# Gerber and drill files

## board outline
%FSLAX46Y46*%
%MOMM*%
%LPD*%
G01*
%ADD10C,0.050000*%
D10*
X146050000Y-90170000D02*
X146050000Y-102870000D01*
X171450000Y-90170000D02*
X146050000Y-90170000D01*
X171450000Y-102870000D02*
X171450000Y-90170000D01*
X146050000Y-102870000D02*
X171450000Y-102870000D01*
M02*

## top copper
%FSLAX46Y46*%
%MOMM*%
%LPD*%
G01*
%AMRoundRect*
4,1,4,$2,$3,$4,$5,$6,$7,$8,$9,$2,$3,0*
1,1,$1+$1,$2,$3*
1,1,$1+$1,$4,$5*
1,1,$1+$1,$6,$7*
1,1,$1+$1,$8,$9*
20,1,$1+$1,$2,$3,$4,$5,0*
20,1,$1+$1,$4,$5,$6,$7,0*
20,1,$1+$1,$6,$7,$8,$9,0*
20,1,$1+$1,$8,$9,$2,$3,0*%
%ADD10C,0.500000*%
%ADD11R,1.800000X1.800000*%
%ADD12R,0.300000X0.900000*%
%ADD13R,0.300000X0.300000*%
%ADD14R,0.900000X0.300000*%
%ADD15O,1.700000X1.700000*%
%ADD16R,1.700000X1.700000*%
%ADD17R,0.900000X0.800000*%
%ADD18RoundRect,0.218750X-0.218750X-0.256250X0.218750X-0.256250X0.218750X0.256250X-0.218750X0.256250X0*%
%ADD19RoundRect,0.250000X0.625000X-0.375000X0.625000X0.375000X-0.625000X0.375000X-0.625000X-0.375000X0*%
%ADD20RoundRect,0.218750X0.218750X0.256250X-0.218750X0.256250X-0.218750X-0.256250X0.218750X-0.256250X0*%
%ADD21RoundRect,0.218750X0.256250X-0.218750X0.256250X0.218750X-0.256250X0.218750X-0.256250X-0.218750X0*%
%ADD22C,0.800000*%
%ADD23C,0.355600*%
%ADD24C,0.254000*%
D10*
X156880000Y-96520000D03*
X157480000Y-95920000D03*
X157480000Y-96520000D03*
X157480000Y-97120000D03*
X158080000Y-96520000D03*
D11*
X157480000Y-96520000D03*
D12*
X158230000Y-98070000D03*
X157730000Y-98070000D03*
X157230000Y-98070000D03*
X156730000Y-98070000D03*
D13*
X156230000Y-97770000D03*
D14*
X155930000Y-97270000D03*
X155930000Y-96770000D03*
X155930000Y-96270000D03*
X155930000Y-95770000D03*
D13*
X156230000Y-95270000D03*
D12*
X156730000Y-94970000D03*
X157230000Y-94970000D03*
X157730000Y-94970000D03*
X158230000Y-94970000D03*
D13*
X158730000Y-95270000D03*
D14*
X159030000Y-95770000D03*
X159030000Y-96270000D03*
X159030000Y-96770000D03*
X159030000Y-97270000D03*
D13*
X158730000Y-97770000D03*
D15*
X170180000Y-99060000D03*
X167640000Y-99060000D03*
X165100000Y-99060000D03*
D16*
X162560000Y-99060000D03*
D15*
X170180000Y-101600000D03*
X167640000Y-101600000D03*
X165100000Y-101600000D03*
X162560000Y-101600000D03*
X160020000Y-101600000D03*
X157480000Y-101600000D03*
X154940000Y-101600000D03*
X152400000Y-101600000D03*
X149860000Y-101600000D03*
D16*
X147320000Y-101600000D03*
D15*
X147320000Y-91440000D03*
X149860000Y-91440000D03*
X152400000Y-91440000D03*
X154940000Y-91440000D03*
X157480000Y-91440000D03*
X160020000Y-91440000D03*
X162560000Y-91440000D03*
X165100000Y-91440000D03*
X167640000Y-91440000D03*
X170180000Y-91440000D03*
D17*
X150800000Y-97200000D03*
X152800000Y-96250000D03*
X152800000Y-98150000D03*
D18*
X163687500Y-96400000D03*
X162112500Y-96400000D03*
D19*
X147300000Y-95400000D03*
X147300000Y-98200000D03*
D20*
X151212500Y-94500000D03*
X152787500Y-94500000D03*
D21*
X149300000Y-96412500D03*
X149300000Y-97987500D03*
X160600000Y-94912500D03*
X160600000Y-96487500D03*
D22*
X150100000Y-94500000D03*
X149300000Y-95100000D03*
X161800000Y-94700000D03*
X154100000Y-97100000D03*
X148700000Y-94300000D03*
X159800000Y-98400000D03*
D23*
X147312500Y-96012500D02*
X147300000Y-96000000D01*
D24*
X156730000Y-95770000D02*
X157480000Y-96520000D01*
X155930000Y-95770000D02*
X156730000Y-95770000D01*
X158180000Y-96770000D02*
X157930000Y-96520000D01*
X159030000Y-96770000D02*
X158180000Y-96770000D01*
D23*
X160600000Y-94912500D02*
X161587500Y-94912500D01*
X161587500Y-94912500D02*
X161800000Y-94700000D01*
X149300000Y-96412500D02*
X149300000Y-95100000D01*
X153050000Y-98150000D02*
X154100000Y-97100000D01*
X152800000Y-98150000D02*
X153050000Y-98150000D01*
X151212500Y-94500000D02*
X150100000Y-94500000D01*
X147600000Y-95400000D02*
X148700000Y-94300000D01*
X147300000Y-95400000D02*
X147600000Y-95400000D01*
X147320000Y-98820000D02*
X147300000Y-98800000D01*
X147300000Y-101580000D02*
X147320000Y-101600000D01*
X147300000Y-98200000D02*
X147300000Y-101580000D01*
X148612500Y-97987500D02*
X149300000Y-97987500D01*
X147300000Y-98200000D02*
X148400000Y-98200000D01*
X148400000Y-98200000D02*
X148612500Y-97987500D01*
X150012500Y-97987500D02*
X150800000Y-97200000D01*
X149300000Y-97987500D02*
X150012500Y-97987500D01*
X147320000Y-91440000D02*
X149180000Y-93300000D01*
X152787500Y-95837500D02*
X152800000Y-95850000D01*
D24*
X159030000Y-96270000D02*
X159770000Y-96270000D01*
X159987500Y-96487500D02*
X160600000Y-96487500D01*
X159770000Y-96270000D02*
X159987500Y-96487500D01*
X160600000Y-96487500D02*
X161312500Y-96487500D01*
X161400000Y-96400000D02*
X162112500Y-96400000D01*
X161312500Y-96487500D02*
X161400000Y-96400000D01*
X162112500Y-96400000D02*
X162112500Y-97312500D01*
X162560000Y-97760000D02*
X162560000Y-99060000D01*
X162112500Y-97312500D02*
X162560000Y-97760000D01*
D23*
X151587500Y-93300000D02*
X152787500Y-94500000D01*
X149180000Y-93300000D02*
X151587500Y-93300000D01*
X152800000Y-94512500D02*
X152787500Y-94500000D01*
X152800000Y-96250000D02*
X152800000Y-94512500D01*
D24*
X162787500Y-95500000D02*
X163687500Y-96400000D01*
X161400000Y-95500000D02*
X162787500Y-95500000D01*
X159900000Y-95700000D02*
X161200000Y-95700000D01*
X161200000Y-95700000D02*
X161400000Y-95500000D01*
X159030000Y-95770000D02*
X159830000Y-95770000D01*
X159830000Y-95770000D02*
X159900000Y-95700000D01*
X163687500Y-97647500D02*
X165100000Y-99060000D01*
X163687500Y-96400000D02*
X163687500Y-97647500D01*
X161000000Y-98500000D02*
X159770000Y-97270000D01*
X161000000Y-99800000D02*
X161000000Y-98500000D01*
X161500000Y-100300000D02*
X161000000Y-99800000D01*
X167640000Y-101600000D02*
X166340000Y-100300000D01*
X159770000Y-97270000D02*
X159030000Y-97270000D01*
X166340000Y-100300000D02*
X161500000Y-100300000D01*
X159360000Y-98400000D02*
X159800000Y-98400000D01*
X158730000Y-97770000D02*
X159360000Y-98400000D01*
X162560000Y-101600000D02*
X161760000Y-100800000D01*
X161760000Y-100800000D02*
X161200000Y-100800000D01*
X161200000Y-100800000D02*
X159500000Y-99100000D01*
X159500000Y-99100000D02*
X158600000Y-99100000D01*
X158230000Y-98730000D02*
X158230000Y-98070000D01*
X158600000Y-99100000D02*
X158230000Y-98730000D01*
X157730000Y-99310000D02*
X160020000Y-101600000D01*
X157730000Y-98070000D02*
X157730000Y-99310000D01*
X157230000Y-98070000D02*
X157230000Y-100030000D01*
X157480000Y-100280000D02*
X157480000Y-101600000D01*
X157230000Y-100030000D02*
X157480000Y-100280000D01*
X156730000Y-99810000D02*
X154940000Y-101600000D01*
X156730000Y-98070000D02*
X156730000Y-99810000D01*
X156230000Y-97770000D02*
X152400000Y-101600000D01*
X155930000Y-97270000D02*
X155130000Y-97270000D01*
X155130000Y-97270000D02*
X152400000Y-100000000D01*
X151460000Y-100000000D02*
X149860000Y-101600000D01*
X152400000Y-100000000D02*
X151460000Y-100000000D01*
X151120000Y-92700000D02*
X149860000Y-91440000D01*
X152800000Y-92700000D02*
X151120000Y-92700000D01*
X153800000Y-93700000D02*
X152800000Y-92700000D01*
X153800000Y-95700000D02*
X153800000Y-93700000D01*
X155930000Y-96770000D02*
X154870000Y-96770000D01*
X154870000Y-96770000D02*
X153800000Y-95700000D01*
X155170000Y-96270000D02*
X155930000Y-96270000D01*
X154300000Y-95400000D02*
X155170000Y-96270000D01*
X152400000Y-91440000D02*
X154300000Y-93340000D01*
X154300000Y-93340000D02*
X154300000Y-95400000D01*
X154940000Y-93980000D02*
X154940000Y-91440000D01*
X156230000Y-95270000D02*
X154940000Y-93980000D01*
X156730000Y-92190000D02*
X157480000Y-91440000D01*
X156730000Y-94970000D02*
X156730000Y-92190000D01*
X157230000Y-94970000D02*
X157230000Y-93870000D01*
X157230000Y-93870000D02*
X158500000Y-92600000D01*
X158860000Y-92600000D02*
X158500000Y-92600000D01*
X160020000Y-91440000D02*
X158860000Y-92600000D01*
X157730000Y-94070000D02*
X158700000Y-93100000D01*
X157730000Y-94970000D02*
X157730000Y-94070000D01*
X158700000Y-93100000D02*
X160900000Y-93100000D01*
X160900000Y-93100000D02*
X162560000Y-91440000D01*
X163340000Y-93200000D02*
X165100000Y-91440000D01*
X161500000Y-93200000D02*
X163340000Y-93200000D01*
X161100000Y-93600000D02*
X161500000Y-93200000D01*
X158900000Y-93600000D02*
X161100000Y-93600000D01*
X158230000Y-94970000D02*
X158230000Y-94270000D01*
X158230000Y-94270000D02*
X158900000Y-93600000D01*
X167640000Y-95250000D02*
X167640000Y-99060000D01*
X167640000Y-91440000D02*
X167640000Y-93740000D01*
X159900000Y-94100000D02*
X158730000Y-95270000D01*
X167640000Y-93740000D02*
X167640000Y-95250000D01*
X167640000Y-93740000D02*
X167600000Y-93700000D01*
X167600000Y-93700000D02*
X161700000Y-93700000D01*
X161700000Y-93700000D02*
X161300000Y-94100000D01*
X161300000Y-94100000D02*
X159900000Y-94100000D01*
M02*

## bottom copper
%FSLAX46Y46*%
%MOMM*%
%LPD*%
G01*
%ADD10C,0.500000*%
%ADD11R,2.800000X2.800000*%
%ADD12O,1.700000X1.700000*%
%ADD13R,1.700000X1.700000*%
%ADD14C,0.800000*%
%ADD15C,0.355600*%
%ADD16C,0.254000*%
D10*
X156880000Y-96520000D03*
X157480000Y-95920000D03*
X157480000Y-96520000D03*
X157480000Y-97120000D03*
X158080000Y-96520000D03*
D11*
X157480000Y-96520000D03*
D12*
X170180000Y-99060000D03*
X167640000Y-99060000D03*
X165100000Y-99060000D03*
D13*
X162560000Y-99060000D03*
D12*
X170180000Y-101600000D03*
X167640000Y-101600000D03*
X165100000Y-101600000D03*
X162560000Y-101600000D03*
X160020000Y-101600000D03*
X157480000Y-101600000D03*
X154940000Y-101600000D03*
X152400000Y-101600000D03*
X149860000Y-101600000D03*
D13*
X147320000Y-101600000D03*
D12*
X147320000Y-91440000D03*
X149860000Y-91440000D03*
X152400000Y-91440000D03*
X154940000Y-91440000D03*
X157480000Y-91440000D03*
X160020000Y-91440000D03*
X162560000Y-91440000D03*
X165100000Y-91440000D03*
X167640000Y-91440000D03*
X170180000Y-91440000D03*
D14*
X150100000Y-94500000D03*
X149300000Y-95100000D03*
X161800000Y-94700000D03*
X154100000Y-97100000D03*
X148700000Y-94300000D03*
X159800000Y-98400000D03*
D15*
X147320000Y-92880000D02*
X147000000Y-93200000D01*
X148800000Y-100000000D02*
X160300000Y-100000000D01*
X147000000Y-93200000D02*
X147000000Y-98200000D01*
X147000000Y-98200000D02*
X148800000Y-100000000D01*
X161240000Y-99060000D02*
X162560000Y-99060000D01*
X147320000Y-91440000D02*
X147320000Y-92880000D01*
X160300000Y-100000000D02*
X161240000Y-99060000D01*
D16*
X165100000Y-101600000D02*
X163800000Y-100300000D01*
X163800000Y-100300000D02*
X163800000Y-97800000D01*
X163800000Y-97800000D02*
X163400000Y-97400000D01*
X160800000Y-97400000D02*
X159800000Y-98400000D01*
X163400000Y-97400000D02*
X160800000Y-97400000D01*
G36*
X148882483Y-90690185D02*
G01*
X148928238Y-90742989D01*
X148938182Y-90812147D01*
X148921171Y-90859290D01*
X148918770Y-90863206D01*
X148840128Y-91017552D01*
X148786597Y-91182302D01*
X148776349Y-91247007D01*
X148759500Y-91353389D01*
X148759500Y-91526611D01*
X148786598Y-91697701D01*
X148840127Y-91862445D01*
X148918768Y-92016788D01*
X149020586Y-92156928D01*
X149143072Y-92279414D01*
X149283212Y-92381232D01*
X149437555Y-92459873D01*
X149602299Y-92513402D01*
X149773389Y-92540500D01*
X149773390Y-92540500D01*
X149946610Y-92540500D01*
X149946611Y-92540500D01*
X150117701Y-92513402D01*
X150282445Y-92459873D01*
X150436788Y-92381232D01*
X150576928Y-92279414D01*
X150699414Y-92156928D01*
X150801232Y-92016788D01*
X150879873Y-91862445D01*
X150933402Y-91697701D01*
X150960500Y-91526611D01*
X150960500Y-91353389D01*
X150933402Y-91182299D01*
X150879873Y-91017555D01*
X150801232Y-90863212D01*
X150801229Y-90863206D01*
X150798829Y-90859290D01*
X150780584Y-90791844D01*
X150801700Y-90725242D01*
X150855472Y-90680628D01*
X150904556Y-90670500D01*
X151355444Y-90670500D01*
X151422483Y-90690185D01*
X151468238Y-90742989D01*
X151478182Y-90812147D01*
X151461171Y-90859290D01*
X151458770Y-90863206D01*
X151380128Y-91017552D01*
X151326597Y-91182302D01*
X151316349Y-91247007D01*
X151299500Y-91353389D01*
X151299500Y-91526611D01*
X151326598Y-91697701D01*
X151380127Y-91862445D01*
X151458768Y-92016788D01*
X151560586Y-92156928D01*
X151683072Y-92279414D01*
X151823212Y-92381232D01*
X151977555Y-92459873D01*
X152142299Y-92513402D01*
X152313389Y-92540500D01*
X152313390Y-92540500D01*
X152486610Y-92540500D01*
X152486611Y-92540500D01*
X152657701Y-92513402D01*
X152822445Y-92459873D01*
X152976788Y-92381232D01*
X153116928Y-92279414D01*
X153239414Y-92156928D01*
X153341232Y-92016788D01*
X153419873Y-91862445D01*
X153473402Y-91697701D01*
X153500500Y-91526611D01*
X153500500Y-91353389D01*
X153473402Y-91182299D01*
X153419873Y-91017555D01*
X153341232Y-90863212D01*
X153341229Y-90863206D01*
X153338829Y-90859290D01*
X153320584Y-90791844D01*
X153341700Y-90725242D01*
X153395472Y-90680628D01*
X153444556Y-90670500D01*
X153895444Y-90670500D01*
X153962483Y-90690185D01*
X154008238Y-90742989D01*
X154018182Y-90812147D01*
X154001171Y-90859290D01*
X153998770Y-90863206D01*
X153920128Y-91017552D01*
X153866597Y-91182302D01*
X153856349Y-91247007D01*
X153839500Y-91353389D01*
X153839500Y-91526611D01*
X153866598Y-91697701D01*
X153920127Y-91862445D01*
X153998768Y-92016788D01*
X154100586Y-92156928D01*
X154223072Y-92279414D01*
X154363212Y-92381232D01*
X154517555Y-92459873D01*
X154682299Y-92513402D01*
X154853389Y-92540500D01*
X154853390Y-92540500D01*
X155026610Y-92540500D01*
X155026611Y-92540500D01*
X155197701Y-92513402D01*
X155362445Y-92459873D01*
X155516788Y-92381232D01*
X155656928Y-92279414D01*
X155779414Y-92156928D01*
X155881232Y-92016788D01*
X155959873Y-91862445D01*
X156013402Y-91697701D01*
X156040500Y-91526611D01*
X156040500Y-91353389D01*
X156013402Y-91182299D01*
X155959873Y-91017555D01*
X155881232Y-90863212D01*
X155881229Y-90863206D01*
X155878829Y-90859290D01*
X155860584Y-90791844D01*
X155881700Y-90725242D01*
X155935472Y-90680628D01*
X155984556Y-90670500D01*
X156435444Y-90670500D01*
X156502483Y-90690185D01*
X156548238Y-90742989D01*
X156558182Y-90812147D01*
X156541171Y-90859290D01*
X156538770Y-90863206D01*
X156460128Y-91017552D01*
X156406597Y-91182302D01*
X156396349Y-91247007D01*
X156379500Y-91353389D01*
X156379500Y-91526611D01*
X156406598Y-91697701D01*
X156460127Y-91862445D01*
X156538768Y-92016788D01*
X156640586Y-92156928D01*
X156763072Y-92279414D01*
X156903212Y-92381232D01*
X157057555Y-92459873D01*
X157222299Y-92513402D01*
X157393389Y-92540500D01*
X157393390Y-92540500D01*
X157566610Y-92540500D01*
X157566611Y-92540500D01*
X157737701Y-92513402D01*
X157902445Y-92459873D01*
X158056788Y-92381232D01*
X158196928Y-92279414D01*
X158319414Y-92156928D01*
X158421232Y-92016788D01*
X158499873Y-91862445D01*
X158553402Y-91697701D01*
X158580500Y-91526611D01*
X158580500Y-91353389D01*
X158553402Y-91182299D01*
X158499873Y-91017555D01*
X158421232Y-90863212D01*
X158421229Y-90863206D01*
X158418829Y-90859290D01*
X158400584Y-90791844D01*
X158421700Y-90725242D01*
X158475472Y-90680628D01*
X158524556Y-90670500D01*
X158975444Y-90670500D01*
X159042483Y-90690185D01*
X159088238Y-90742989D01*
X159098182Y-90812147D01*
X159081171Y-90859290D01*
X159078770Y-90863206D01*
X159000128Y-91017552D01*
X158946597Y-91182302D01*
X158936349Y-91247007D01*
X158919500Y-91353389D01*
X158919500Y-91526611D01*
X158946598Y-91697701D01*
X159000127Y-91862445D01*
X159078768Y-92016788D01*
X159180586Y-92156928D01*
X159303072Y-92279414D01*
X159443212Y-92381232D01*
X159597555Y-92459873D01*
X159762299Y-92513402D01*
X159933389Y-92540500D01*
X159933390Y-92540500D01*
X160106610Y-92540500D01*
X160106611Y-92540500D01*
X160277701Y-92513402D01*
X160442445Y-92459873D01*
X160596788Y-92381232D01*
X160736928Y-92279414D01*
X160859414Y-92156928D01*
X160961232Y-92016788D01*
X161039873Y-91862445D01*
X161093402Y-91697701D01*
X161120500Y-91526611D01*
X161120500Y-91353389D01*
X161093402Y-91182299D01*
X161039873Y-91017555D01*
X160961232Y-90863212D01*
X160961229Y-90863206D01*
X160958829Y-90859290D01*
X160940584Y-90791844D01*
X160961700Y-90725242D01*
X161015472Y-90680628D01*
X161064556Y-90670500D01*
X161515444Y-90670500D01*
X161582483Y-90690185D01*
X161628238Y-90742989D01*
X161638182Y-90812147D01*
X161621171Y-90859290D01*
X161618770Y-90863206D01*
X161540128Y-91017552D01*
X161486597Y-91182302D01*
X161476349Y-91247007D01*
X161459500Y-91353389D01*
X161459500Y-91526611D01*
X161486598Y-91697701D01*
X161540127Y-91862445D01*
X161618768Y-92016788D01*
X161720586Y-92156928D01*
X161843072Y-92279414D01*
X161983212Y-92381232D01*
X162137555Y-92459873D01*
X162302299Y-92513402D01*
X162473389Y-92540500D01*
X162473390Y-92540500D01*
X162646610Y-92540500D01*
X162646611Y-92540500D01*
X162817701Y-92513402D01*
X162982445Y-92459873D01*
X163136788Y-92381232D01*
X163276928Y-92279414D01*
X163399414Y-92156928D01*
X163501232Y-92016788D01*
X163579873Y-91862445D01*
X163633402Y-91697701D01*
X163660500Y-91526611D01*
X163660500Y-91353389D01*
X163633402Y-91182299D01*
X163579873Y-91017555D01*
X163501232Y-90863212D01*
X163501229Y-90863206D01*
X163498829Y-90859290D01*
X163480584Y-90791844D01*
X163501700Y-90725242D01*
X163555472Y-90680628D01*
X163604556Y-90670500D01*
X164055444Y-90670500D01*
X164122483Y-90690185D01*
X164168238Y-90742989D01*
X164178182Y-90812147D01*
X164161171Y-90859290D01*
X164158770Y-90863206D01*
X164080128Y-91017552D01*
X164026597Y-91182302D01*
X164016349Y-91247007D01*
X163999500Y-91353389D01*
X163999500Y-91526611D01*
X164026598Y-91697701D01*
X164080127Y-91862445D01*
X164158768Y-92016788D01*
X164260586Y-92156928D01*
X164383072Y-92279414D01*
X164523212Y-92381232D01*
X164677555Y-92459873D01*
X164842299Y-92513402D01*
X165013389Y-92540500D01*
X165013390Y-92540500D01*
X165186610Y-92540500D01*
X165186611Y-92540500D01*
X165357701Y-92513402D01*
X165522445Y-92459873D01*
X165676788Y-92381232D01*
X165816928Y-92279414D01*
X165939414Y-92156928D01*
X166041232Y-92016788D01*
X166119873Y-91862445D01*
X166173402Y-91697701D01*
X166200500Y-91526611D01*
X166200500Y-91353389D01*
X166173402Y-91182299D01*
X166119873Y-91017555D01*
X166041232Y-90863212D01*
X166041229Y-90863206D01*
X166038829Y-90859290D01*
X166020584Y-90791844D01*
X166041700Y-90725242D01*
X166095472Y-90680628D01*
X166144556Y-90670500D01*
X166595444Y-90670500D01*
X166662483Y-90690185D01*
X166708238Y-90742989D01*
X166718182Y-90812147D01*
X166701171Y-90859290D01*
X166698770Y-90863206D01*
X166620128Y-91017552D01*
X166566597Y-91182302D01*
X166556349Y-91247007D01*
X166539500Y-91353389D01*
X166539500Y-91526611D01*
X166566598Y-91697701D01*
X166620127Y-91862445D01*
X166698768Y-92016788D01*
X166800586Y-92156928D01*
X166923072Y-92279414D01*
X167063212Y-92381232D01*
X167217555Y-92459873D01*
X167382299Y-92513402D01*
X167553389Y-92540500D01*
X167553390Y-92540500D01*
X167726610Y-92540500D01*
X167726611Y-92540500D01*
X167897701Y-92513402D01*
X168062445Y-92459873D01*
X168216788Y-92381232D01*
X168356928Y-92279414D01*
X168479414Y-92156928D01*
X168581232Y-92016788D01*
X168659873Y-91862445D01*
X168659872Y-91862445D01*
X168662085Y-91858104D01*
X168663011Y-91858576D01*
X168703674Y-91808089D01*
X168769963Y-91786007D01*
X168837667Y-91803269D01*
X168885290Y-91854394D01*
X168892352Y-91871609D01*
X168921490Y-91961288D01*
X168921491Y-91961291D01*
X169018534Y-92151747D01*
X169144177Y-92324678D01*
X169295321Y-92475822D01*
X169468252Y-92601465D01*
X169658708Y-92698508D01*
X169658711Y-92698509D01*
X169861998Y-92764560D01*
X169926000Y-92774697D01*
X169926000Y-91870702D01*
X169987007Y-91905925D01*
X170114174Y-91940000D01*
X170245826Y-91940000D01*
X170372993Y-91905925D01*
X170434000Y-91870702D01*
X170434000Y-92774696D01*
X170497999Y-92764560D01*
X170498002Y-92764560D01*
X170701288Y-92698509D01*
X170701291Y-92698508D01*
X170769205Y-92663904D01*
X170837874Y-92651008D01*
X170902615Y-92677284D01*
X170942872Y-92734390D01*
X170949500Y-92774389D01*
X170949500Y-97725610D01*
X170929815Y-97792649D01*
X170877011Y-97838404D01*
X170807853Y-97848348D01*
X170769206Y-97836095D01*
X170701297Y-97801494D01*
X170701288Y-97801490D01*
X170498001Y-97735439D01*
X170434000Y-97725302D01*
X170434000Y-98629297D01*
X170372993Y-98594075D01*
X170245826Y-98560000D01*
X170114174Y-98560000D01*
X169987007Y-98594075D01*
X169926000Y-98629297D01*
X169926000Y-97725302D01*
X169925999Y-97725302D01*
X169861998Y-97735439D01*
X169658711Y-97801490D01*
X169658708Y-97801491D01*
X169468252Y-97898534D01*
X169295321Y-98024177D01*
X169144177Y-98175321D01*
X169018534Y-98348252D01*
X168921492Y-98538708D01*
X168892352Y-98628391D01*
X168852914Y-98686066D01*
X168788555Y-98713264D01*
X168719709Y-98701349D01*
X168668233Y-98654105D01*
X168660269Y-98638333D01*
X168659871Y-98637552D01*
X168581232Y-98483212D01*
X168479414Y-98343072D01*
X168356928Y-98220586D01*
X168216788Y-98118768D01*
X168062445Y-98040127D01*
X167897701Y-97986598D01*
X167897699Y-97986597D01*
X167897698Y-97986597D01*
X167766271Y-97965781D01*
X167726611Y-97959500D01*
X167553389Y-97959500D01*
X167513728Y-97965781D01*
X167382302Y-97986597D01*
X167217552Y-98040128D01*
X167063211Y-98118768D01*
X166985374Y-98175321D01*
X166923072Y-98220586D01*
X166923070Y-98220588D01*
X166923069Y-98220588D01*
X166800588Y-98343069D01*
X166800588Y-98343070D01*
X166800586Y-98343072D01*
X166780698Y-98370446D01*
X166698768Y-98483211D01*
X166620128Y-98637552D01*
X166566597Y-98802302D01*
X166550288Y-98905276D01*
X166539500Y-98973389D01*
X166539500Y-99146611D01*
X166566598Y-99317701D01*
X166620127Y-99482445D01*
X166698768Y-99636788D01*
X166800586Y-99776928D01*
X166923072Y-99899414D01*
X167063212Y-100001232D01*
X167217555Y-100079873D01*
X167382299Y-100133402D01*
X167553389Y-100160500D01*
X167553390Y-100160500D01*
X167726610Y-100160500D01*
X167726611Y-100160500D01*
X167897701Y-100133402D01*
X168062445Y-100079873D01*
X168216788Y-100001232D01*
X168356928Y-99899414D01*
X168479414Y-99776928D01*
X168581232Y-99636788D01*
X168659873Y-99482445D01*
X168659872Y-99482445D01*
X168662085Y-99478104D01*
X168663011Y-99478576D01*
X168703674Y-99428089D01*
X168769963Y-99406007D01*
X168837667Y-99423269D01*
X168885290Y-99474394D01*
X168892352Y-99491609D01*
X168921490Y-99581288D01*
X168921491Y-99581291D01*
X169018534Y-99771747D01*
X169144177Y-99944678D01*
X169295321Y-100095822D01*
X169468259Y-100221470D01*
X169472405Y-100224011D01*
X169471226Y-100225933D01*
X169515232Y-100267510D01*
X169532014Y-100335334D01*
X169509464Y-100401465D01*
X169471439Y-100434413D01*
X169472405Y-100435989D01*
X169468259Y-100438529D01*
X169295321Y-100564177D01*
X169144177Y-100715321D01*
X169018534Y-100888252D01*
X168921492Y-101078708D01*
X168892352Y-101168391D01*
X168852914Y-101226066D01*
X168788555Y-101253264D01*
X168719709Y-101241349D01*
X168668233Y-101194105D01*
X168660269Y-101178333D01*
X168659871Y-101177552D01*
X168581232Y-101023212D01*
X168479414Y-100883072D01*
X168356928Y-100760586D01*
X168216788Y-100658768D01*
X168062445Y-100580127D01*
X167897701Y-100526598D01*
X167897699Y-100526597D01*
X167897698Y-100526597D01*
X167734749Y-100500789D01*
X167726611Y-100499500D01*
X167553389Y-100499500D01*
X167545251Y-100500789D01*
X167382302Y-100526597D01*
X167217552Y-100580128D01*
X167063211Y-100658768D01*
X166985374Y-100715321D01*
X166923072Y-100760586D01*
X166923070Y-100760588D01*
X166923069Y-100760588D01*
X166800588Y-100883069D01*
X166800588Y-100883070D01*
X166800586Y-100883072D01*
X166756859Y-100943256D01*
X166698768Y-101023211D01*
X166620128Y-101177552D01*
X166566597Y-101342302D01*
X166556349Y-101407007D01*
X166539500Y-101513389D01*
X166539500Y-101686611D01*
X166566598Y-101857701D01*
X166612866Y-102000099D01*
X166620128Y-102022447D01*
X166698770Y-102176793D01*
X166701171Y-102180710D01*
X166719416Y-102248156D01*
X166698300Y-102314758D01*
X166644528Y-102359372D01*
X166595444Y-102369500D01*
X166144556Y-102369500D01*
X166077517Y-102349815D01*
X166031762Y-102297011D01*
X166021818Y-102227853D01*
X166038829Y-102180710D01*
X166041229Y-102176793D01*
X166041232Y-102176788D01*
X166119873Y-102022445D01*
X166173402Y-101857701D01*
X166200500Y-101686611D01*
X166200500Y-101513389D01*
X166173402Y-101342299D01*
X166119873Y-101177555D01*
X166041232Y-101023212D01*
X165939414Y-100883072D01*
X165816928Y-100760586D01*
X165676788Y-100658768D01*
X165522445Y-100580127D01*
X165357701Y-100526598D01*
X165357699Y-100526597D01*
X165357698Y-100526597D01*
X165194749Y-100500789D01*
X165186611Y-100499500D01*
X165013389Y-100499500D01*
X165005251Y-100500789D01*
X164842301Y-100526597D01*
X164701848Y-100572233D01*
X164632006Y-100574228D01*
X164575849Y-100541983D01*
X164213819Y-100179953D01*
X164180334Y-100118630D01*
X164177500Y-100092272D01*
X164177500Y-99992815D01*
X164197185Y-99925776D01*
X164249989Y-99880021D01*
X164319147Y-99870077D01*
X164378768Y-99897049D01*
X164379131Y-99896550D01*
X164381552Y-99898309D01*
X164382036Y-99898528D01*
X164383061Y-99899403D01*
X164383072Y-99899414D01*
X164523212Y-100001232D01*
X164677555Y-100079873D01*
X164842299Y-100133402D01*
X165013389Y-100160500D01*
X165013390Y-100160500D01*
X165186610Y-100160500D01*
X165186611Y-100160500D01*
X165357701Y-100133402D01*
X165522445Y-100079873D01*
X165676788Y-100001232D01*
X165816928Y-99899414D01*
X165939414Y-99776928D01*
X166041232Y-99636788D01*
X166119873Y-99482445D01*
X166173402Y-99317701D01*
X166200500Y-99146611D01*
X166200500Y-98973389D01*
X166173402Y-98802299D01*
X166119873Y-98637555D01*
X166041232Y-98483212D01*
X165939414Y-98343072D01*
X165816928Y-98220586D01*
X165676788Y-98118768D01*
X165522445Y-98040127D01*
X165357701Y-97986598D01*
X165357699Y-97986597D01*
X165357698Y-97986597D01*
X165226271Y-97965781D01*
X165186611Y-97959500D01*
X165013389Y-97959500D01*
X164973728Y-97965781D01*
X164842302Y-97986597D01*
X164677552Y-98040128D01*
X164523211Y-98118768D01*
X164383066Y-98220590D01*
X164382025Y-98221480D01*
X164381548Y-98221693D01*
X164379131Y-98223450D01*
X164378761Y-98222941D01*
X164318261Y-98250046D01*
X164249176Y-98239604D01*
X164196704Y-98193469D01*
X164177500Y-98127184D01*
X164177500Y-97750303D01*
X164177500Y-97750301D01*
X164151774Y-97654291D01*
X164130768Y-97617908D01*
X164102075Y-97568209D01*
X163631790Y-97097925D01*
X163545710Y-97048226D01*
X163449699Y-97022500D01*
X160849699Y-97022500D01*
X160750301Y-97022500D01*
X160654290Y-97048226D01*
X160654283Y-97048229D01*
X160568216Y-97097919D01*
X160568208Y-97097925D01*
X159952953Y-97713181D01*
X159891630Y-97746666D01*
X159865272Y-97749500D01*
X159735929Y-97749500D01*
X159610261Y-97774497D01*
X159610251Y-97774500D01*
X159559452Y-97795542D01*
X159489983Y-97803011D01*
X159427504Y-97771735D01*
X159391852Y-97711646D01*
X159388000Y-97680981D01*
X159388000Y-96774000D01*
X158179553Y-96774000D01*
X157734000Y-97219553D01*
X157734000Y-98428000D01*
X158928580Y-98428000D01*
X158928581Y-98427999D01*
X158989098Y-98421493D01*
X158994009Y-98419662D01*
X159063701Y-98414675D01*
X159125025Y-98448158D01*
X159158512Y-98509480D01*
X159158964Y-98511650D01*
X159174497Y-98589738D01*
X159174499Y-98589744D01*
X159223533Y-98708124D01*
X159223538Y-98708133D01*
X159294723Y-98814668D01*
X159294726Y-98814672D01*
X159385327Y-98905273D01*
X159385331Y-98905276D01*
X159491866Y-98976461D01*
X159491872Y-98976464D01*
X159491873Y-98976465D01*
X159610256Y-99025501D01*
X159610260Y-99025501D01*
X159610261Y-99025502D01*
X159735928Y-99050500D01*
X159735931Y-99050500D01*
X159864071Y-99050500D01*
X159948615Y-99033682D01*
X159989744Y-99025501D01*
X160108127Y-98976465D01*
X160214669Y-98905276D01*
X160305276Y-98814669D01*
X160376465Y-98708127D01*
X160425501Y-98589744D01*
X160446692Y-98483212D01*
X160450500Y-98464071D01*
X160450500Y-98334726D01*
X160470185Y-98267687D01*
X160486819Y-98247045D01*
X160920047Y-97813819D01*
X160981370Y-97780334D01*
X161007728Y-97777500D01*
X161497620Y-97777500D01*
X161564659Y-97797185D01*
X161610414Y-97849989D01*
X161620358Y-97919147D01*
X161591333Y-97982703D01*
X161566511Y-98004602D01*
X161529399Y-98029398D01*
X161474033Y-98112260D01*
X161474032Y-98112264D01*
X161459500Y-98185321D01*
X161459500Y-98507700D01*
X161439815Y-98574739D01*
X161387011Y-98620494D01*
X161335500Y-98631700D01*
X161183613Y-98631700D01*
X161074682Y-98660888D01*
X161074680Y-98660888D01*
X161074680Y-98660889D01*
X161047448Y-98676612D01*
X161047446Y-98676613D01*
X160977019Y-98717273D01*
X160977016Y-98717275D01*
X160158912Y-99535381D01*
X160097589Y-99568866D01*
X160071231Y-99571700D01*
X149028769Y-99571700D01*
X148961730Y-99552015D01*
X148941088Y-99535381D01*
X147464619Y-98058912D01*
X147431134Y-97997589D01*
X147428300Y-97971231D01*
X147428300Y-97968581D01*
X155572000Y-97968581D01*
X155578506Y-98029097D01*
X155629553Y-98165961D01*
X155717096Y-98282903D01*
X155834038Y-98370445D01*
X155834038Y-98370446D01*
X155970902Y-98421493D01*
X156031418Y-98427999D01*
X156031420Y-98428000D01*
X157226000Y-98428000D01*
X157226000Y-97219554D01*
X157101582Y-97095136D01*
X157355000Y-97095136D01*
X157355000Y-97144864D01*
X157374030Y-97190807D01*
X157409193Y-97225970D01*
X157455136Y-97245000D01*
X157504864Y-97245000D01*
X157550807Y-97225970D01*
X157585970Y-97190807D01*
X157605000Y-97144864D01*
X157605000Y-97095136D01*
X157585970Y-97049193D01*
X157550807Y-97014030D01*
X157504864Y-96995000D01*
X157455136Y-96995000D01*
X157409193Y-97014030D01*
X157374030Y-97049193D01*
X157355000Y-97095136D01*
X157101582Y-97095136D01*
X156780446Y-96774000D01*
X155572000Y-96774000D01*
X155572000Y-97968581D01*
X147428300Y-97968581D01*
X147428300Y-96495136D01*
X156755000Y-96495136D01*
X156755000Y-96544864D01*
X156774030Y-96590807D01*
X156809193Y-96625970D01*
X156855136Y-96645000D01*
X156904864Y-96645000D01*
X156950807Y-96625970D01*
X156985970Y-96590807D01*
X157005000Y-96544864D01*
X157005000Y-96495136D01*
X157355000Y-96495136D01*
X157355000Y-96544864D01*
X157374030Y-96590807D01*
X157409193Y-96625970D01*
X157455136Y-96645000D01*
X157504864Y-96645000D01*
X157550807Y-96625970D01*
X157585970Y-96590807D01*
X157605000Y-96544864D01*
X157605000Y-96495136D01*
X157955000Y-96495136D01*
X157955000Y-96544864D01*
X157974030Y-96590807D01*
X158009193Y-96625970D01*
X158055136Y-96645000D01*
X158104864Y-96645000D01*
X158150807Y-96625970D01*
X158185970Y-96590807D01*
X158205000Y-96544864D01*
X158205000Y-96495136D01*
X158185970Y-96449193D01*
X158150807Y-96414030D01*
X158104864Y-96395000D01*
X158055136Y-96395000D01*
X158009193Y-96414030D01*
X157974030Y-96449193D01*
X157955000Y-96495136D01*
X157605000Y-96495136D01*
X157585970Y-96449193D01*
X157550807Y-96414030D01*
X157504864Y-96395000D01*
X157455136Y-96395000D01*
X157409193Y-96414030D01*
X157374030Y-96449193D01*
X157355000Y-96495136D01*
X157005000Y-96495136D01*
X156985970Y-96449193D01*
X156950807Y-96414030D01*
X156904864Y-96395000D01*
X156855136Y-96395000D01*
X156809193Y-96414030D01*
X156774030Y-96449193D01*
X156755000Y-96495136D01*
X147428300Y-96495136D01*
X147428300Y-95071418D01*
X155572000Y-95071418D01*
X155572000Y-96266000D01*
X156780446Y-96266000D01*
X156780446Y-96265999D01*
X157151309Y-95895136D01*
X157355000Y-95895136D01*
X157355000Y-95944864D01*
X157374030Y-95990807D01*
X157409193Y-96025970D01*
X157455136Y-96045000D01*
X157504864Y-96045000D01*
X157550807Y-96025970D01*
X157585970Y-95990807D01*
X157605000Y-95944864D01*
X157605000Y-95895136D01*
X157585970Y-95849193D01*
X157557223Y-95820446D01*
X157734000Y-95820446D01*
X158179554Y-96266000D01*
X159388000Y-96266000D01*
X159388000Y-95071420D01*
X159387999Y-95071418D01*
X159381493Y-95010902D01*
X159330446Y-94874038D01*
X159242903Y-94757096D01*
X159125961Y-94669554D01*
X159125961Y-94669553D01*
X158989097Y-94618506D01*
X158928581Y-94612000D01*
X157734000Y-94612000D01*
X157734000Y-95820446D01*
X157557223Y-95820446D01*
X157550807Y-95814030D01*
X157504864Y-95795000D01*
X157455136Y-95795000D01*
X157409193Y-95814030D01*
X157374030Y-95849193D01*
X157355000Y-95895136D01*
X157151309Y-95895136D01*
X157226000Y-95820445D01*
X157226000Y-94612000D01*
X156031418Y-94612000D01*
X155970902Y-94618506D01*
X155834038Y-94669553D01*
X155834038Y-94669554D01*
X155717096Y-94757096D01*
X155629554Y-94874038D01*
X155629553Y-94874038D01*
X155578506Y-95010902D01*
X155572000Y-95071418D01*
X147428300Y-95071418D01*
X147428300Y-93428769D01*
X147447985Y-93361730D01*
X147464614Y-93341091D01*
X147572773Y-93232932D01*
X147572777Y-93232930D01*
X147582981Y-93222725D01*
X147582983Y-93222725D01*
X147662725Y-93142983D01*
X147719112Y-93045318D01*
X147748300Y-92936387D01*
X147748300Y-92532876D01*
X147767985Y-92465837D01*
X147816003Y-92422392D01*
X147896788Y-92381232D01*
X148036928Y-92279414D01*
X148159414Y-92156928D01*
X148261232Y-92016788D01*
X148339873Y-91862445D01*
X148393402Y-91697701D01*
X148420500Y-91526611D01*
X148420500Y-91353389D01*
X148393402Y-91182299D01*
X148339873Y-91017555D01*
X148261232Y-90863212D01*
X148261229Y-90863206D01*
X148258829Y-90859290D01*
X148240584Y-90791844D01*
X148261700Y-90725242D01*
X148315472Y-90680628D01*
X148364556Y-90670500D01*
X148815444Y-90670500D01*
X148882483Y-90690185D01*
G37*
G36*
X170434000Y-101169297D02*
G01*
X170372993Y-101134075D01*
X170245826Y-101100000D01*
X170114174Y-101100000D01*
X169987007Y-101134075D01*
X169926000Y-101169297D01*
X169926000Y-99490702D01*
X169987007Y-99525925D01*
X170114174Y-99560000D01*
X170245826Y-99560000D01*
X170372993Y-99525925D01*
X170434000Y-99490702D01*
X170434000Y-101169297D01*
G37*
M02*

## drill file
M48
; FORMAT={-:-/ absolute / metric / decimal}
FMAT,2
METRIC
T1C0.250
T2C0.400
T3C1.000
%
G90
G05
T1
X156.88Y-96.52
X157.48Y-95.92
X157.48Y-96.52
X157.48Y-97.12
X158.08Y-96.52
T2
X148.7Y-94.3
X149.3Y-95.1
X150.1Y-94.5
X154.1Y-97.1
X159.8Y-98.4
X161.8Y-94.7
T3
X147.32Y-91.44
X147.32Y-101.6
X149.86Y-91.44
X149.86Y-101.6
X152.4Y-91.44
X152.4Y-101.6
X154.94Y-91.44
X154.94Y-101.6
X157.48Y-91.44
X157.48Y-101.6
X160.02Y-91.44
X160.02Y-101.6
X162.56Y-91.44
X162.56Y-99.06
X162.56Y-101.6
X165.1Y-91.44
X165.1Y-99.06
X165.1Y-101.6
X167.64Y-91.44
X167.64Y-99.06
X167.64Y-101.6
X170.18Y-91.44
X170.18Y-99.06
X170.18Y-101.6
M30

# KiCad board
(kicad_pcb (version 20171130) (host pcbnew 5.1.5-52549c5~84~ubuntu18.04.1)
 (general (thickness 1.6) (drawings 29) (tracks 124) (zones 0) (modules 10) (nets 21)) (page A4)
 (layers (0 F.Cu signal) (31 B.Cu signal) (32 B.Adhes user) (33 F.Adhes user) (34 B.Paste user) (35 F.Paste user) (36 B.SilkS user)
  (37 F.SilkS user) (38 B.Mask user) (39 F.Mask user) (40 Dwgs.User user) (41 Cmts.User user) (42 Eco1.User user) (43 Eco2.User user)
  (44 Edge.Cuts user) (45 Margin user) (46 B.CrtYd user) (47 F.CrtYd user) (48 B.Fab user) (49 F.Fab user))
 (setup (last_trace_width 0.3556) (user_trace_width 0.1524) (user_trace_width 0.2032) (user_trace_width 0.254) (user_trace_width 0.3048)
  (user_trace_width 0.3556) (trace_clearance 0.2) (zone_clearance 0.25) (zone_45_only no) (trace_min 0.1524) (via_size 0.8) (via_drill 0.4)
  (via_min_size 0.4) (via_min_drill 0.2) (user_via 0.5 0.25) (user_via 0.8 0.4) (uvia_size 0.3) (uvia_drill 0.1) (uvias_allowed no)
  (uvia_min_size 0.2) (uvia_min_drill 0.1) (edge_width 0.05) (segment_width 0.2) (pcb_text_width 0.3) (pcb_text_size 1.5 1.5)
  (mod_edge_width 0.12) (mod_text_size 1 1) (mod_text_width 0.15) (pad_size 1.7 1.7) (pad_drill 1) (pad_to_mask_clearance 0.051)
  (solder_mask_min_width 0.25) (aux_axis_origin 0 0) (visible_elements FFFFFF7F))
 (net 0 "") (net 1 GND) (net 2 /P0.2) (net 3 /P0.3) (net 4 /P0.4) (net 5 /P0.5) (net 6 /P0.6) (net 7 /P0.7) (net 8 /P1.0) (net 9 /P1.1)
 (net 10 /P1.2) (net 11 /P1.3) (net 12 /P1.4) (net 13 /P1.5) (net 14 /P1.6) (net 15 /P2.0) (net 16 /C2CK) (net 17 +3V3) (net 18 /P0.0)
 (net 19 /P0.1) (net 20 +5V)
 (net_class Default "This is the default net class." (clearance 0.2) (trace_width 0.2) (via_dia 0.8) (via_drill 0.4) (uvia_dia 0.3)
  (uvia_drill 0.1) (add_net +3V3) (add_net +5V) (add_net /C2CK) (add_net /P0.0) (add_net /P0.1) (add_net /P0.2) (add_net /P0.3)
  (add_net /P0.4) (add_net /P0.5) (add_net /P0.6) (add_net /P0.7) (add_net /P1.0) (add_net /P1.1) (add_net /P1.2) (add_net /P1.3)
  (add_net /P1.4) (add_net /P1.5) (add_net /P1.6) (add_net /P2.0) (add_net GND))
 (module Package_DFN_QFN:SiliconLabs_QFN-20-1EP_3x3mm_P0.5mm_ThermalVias (layer F.Cu) (at 157.48 96.52 180)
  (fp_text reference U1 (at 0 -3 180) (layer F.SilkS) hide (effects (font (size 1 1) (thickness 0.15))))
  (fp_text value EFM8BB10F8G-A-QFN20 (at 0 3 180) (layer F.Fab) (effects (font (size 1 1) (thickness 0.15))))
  (pad 21 thru_hole circle (at 0.6 0 180) (size 0.5 0.5) (drill 0.25) (layers *.Cu) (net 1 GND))
  (pad 21 thru_hole circle (at 0 0.6 180) (size 0.5 0.5) (drill 0.25) (layers *.Cu) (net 1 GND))
  (pad 21 thru_hole circle (at 0 0 180) (size 0.5 0.5) (drill 0.25) (layers *.Cu) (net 1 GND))
  (pad 21 thru_hole circle (at 0 -0.6 180) (size 0.5 0.5) (drill 0.25) (layers *.Cu) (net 1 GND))
  (pad 21 thru_hole circle (at -0.6 0 180) (size 0.5 0.5) (drill 0.25) (layers *.Cu) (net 1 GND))
  (pad "" smd rect (at 0.45 0.45 180) (size 0.54 0.54) (layers F.Paste))
  (pad "" smd rect (at 0.45 -0.45 180) (size 0.54 0.54) (layers F.Paste))
  (pad "" smd rect (at -0.45 0.45 180) (size 0.54 0.54) (layers F.Paste))
  (pad "" smd rect (at -0.45 -0.45 180) (size 0.54 0.54) (layers F.Paste))
  (pad 21 smd rect (at 0 0 180) (size 1.8 1.8) (layers F.Cu F.Mask) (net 1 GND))
  (pad 21 smd rect (at 0 0 180) (size 2.8 2.8) (layers B.Cu) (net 1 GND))
  (pad 20 smd rect (at -0.75 -1.55 270) (size 0.9 0.3) (layers F.Cu F.Paste F.Mask) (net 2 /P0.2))
  (pad 19 smd rect (at -0.25 -1.55 270) (size 0.9 0.3) (layers F.Cu F.Paste F.Mask) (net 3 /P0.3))
  (pad 18 smd rect (at 0.25 -1.55 270) (size 0.9 0.3) (layers F.Cu F.Paste F.Mask) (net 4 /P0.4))
  (pad 17 smd rect (at 0.75 -1.55 270) (size 0.9 0.3) (layers F.Cu F.Paste F.Mask) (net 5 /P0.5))
  (pad 16 smd rect (at 1.25 -1.25 180) (size 0.3 0.3) (layers F.Cu F.Paste F.Mask) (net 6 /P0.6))
  (pad 15 smd rect (at 1.55 -0.75 180) (size 0.9 0.3) (layers F.Cu F.Paste F.Mask) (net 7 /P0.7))
  (pad 14 smd rect (at 1.55 -0.25 180) (size 0.9 0.3) (layers F.Cu F.Paste F.Mask) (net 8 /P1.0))
  (pad 13 smd rect (at 1.55 0.25 180) (size 0.9 0.3) (layers F.Cu F.Paste F.Mask) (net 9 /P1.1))
  (pad 12 smd rect (at 1.55 0.75 180) (size 0.9 0.3) (layers F.Cu F.Paste F.Mask) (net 1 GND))
  (pad 11 smd rect (at 1.25 1.25 180) (size 0.3 0.3) (layers F.Cu F.Paste F.Mask) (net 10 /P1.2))
  (pad 10 smd rect (at 0.75 1.55 270) (size 0.9 0.3) (layers F.Cu F.Paste F.Mask) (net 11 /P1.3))
  (pad 9 smd rect (at 0.25 1.55 270) (size 0.9 0.3) (layers F.Cu F.Paste F.Mask) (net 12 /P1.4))
  (pad 8 smd rect (at -0.25 1.55 270) (size 0.9 0.3) (layers F.Cu F.Paste F.Mask) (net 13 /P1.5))
  (pad 7 smd rect (at -0.75 1.55 270) (size 0.9 0.3) (layers F.Cu F.Paste F.Mask) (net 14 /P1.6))
  (pad 6 smd rect (at -1.25 1.25 180) (size 0.3 0.3) (layers F.Cu F.Paste F.Mask) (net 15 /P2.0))
  (pad 5 smd rect (at -1.55 0.75 180) (size 0.9 0.3) (layers F.Cu F.Paste F.Mask) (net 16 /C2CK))
  (pad 4 smd rect (at -1.55 0.25 180) (size 0.9 0.3) (layers F.Cu F.Paste F.Mask) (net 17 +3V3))
  (pad 3 smd rect (at -1.55 -0.25 180) (size 0.9 0.3) (layers F.Cu F.Paste F.Mask) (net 1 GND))
  (pad 2 smd rect (at -1.55 -0.75 180) (size 0.9 0.3) (layers F.Cu F.Paste F.Mask) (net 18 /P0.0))
  (pad 1 smd rect (at -1.25 -1.25 180) (size 0.3 0.3) (layers F.Cu F.Paste F.Mask) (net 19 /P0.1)))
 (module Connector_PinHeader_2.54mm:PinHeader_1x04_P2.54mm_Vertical (layer F.Cu) (at 162.56 99.06 90)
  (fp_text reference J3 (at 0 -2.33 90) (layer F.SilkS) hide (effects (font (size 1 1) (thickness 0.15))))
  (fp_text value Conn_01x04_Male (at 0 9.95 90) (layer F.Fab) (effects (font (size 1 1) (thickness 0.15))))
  (pad 4 thru_hole oval (at 0 7.62 90) (size 1.7 1.7) (drill 1) (layers *.Cu *.Mask) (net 1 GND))
  (pad 3 thru_hole oval (at 0 5.08 90) (size 1.7 1.7) (drill 1) (layers *.Cu *.Mask) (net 15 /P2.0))
  (pad 2 thru_hole oval (at 0 2.54 90) (size 1.7 1.7) (drill 1) (layers *.Cu *.Mask) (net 16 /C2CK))
  (pad 1 thru_hole rect (at 0 0 90) (size 1.7 1.7) (drill 1) (layers *.Cu *.Mask) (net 17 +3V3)))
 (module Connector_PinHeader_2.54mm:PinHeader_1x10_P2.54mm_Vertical (layer F.Cu) (at 147.32 101.6 90)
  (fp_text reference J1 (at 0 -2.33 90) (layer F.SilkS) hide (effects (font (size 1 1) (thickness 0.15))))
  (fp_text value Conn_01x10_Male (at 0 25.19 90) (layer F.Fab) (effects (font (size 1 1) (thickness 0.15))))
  (pad 10 thru_hole oval (at 0 22.86 90) (size 1.7 1.7) (drill 1) (layers *.Cu *.Mask) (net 1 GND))
  (pad 9 thru_hole oval (at 0 20.32 90) (size 1.7 1.7) (drill 1) (layers *.Cu *.Mask) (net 18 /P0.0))
  (pad 8 thru_hole oval (at 0 17.78 90) (size 1.7 1.7) (drill 1) (layers *.Cu *.Mask) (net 19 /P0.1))
  (pad 7 thru_hole oval (at 0 15.24 90) (size 1.7 1.7) (drill 1) (layers *.Cu *.Mask) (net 2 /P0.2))
  (pad 6 thru_hole oval (at 0 12.7 90) (size 1.7 1.7) (drill 1) (layers *.Cu *.Mask) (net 3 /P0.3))
  (pad 5 thru_hole oval (at 0 10.16 90) (size 1.7 1.7) (drill 1) (layers *.Cu *.Mask) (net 4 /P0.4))
  (pad 4 thru_hole oval (at 0 7.62 90) (size 1.7 1.7) (drill 1) (layers *.Cu *.Mask) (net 5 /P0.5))
  (pad 3 thru_hole oval (at 0 5.08 90) (size 1.7 1.7) (drill 1) (layers *.Cu *.Mask) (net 6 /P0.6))
  (pad 2 thru_hole oval (at 0 2.54 90) (size 1.7 1.7) (drill 1) (layers *.Cu *.Mask) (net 7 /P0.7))
  (pad 1 thru_hole rect (at 0 0 90) (size 1.7 1.7) (drill 1) (layers *.Cu *.Mask) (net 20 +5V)))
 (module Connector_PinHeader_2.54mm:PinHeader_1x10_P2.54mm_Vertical (layer F.Cu) (at 170.18 91.44 270)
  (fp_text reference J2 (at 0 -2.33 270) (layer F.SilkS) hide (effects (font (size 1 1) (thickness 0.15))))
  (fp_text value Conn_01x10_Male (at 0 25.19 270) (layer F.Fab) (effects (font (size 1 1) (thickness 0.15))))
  (pad 10 thru_hole oval (at 0 22.86 270) (size 1.7 1.7) (drill 1) (layers *.Cu *.Mask) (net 17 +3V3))
  (pad 9 thru_hole oval (at 0 20.32 270) (size 1.7 1.7) (drill 1) (layers *.Cu *.Mask) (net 8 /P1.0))
  (pad 8 thru_hole oval (at 0 17.78 270) (size 1.7 1.7) (drill 1) (layers *.Cu *.Mask) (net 9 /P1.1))
  (pad 7 thru_hole oval (at 0 15.24 270) (size 1.7 1.7) (drill 1) (layers *.Cu *.Mask) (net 10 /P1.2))
  (pad 6 thru_hole oval (at 0 12.7 270) (size 1.7 1.7) (drill 1) (layers *.Cu *.Mask) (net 11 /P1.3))
  (pad 5 thru_hole oval (at 0 10.16 270) (size 1.7 1.7) (drill 1) (layers *.Cu *.Mask) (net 12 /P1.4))
  (pad 4 thru_hole oval (at 0 7.62 270) (size 1.7 1.7) (drill 1) (layers *.Cu *.Mask) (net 13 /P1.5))
  (pad 3 thru_hole oval (at 0 5.08 270) (size 1.7 1.7) (drill 1) (layers *.Cu *.Mask) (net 14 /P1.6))
  (pad 2 thru_hole oval (at 0 2.54 270) (size 1.7 1.7) (drill 1) (layers *.Cu *.Mask) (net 15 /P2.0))
  (pad 1 thru_hole oval (at 0 0 270) (size 1.7 1.7) (drill 1) (layers *.Cu *.Mask) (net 1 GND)))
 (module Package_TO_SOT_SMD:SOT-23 (layer F.Cu) (at 151.8 97.2 180)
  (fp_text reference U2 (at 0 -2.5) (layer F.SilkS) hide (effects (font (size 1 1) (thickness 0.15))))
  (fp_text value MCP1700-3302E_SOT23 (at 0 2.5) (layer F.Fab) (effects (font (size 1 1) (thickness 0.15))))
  (pad 3 smd rect (at 1 0 180) (size 0.9 0.8) (layers F.Cu F.Paste F.Mask) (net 20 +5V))
  (pad 2 smd rect (at -1 0.95 180) (size 0.9 0.8) (layers F.Cu F.Paste F.Mask) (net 17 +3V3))
  (pad 1 smd rect (at -1 -0.95 180) (size 0.9 0.8) (layers F.Cu F.Paste F.Mask) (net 1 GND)))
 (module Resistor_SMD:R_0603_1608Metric (layer F.Cu) (at 162.9 96.4)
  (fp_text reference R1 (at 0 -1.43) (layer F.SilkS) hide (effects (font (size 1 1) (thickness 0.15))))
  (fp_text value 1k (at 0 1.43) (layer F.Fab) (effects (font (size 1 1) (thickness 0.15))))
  (pad 2 smd roundrect (at 0.7875 0) (size 0.875 0.95) (layers F.Cu F.Paste F.Mask) (roundrect_rratio 0.25) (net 16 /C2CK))
  (pad 1 smd roundrect (at -0.7875 0) (size 0.875 0.95) (layers F.Cu F.Paste F.Mask) (roundrect_rratio 0.25) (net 17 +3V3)))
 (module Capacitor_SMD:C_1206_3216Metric (layer F.Cu) (at 147.3 96.8 90)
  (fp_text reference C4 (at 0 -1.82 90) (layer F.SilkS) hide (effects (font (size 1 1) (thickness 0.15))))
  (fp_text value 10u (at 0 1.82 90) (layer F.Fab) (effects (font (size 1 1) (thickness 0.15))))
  (pad 2 smd roundrect (at 1.4 0 90) (size 1.25 1.75) (layers F.Cu F.Paste F.Mask) (roundrect_rratio 0.2) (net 1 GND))
  (pad 1 smd roundrect (at -1.4 0 90) (size 1.25 1.75) (layers F.Cu F.Paste F.Mask) (roundrect_rratio 0.2) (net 20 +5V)))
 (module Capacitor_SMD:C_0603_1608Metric (layer F.Cu) (at 152 94.5 180)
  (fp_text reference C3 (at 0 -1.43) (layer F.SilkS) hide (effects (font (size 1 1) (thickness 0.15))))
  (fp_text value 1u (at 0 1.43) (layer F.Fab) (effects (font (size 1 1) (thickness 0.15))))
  (pad 2 smd roundrect (at 0.7875 0 180) (size 0.875 0.95) (layers F.Cu F.Paste F.Mask) (roundrect_rratio 0.25) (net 1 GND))
  (pad 1 smd roundrect (at -0.7875 0 180) (size 0.875 0.95) (layers F.Cu F.Paste F.Mask) (roundrect_rratio 0.25) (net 17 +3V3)))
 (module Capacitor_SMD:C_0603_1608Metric (layer F.Cu) (at 149.3 97.2 90)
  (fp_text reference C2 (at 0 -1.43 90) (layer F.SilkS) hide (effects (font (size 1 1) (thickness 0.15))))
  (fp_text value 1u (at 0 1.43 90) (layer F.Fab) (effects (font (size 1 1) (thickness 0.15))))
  (pad 2 smd roundrect (at 0.7875 0 90) (size 0.875 0.95) (layers F.Cu F.Paste F.Mask) (roundrect_rratio 0.25) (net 1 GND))
  (pad 1 smd roundrect (at -0.7875 0 90) (size 0.875 0.95) (layers F.Cu F.Paste F.Mask) (roundrect_rratio 0.25) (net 20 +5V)))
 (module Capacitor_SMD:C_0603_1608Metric (layer F.Cu) (at 160.6 95.7 90)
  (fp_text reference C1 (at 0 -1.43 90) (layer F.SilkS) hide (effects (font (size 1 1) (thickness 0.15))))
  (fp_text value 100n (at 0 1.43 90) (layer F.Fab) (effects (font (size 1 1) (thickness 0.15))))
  (pad 2 smd roundrect (at 0.7875 0 90) (size 0.875 0.95) (layers F.Cu F.Paste F.Mask) (roundrect_rratio 0.25) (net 1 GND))
  (pad 1 smd roundrect (at -0.7875 0 90) (size 0.875 0.95) (layers F.Cu F.Paste F.Mask) (roundrect_rratio 0.25) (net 17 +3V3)))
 (gr_line (start 146.05 90.17) (end 146.05 102.87) (layer Edge.Cuts) (width 0.05))
 (gr_line (start 171.45 90.17) (end 146.05 90.17) (layer Edge.Cuts) (width 0.05))
 (gr_line (start 171.45 102.87) (end 171.45 90.17) (layer Edge.Cuts) (width 0.05))
 (gr_line (start 146.05 102.87) (end 171.45 102.87) (layer Edge.Cuts) (width 0.05))
 (segment (start 147.3125 96.0125) (end 147.3 96) (width 0.3556) (layer F.Cu) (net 1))
 (via (at 150.1 94.5) (size 0.8) (drill 0.4) (layers F.Cu B.Cu) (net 1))
 (via (at 149.3 95.1) (size 0.8) (drill 0.4) (layers F.Cu B.Cu) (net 1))
 (segment (start 156.73 95.77) (end 157.48 96.52) (width 0.254) (layer F.Cu) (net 1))
 (segment (start 155.93 95.77) (end 156.73 95.77) (width 0.254) (layer F.Cu) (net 1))
 (segment (start 158.18 96.77) (end 157.93 96.52) (width 0.254) (layer F.Cu) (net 1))
 (segment (start 159.03 96.77) (end 158.18 96.77) (width 0.254) (layer F.Cu) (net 1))
 (segment (start 160.6 94.9125) (end 161.5875 94.9125) (width 0.3556) (layer F.Cu) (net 1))
 (via (at 161.8 94.7) (size 0.8) (drill 0.4) (layers F.Cu B.Cu) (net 1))
 (segment (start 161.5875 94.9125) (end 161.8 94.7) (width 0.3556) (layer F.Cu) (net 1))
 (via (at 154.1 97.1) (size 0.8) (drill 0.4) (layers F.Cu B.Cu) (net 1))
 (via (at 148.7 94.3) (size 0.8) (drill 0.4) (layers F.Cu B.Cu) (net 1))
 (segment (start 149.3 96.4125) (end 149.3 95.1) (width 0.3556) (layer F.Cu) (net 1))
 (segment (start 153.05 98.15) (end 154.1 97.1) (width 0.3556) (layer F.Cu) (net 1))
 (segment (start 152.8 98.15) (end 153.05 98.15) (width 0.3556) (layer F.Cu) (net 1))
 (segment (start 151.2125 94.5) (end 150.1 94.5) (width 0.3556) (layer F.Cu) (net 1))
 (segment (start 147.6 95.4) (end 148.7 94.3) (width 0.3556) (layer F.Cu) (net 1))
 (segment (start 147.3 95.4) (end 147.6 95.4) (width 0.3556) (layer F.Cu) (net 1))
 (via (at 159.8 98.4) (size 0.8) (drill 0.4) (layers F.Cu B.Cu) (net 19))
 (segment (start 147.32 98.82) (end 147.3 98.8) (width 0.3556) (layer F.Cu) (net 20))
 (segment (start 147.3 101.58) (end 147.32 101.6) (width 0.3556) (layer F.Cu) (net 20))
 (segment (start 147.3 98.2) (end 147.3 101.58) (width 0.3556) (layer F.Cu) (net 20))
 (segment (start 148.6125 97.9875) (end 149.3 97.9875) (width 0.3556) (layer F.Cu) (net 20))
 (segment (start 147.3 98.2) (end 148.4 98.2) (width 0.3556) (layer F.Cu) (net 20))
 (segment (start 148.4 98.2) (end 148.6125 97.9875) (width 0.3556) (layer F.Cu) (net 20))
 (segment (start 150.0125 97.9875) (end 150.8 97.2) (width 0.3556) (layer F.Cu) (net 20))
 (segment (start 149.3 97.9875) (end 150.0125 97.9875) (width 0.3556) (layer F.Cu) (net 20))
 (segment (start 147.32 91.44) (end 149.18 93.3) (width 0.3556) (layer F.Cu) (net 17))
 (segment (start 152.7875 95.8375) (end 152.8 95.85) (width 0.3556) (layer F.Cu) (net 17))
 (segment (start 159.03 96.27) (end 159.77 96.27) (width 0.254) (layer F.Cu) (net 17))
 (segment (start 159.9875 96.4875) (end 160.6 96.4875) (width 0.254) (layer F.Cu) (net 17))
 (segment (start 159.77 96.27) (end 159.9875 96.4875) (width 0.254) (layer F.Cu) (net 17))
 (segment (start 160.6 96.4875) (end 161.3125 96.4875) (width 0.254) (layer F.Cu) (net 17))
 (segment (start 161.4 96.4) (end 162.1125 96.4) (width 0.254) (layer F.Cu) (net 17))
 (segment (start 161.3125 96.4875) (end 161.4 96.4) (width 0.254) (layer F.Cu) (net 17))
 (segment (start 162.1125 96.4) (end 162.1125 97.3125) (width 0.254) (layer F.Cu) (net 17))
 (segment (start 162.56 97.76) (end 162.56 99.06) (width 0.254) (layer F.Cu) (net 17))
 (segment (start 162.1125 97.3125) (end 162.56 97.76) (width 0.254) (layer F.Cu) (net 17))
 (segment (start 147.32 92.88) (end 147 93.2) (width 0.3556) (layer B.Cu) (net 17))
 (segment (start 148.8 100) (end 160.3 100) (width 0.3556) (layer B.Cu) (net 17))
 (segment (start 147 93.2) (end 147 98.2) (width 0.3556) (layer B.Cu) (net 17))
 (segment (start 147 98.2) (end 148.8 100) (width 0.3556) (layer B.Cu) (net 17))
 (segment (start 161.24 99.06) (end 162.56 99.06) (width 0.3556) (layer B.Cu) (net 17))
 (segment (start 147.32 91.44) (end 147.32 92.88) (width 0.3556) (layer B.Cu) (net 17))
 (segment (start 160.3 100) (end 161.24 99.06) (width 0.3556) (layer B.Cu) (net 17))
 (segment (start 151.5875 93.3) (end 152.7875 94.5) (width 0.3556) (layer F.Cu) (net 17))
 (segment (start 149.18 93.3) (end 151.5875 93.3) (width 0.3556) (layer F.Cu) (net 17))
 (segment (start 152.8 94.5125) (end 152.7875 94.5) (width 0.3556) (layer F.Cu) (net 17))
 (segment (start 152.8 96.25) (end 152.8 94.5125) (width 0.3556) (layer F.Cu) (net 17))
 (segment (start 162.7875 95.5) (end 163.6875 96.4) (width 0.254) (layer F.Cu) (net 16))
 (segment (start 161.4 95.5) (end 162.7875 95.5) (width 0.254) (layer F.Cu) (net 16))
 (segment (start 159.9 95.7) (end 161.2 95.7) (width 0.254) (layer F.Cu) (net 16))
 (segment (start 161.2 95.7) (end 161.4 95.5) (width 0.254) (layer F.Cu) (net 16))
 (segment (start 159.03 95.77) (end 159.83 95.77) (width 0.254) (layer F.Cu) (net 16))
 (segment (start 159.83 95.77) (end 159.9 95.7) (width 0.254) (layer F.Cu) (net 16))
 (segment (start 163.6875 97.6475) (end 165.1 99.06) (width 0.254) (layer F.Cu) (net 16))
 (segment (start 163.6875 96.4) (end 163.6875 97.6475) (width 0.254) (layer F.Cu) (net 16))
 (segment (start 161 98.5) (end 159.77 97.27) (width 0.254) (layer F.Cu) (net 18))
 (segment (start 161 99.8) (end 161 98.5) (width 0.254) (layer F.Cu) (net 18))
 (segment (start 161.5 100.3) (end 161 99.8) (width 0.254) (layer F.Cu) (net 18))
 (segment (start 167.64 101.6) (end 166.34 100.3) (width 0.254) (layer F.Cu) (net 18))
 (segment (start 159.77 97.27) (end 159.03 97.27) (width 0.254) (layer F.Cu) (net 18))
 (segment (start 166.34 100.3) (end 161.5 100.3) (width 0.254) (layer F.Cu) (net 18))
 (segment (start 159.36 98.4) (end 159.8 98.4) (width 0.254) (layer F.Cu) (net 19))
 (segment (start 158.73 97.77) (end 159.36 98.4) (width 0.254) (layer F.Cu) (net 19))
 (segment (start 165.1 101.6) (end 163.8 100.3) (width 0.254) (layer B.Cu) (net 19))
 (segment (start 163.8 100.3) (end 163.8 97.8) (width 0.254) (layer B.Cu) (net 19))
 (segment (start 163.8 97.8) (end 163.4 97.4) (width 0.254) (layer B.Cu) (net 19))
 (segment (start 160.8 97.4) (end 159.8 98.4) (width 0.254) (layer B.Cu) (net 19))
 (segment (start 163.4 97.4) (end 160.8 97.4) (width 0.254) (layer B.Cu) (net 19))
 (segment (start 162.56 101.6) (end 161.76 100.8) (width 0.254) (layer F.Cu) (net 2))
 (segment (start 161.76 100.8) (end 161.2 100.8) (width 0.254) (layer F.Cu) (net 2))
 (segment (start 161.2 100.8) (end 159.5 99.1) (width 0.254) (layer F.Cu) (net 2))
 (segment (start 159.5 99.1) (end 158.6 99.1) (width 0.254) (layer F.Cu) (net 2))
 (segment (start 158.23 98.73) (end 158.23 98.07) (width 0.254) (layer F.Cu) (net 2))
 (segment (start 158.6 99.1) (end 158.23 98.73) (width 0.254) (layer F.Cu) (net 2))
 (segment (start 157.73 99.31) (end 160.02 101.6) (width 0.254) (layer F.Cu) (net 3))
 (segment (start 157.73 98.07) (end 157.73 99.31) (width 0.254) (layer F.Cu) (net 3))
 (segment (start 157.23 98.07) (end 157.23 100.03) (width 0.254) (layer F.Cu) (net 4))
 (segment (start 157.48 100.28) (end 157.48 101.6) (width 0.254) (layer F.Cu) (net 4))
 (segment (start 157.23 100.03) (end 157.48 100.28) (width 0.254) (layer F.Cu) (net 4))
 (segment (start 156.73 99.81) (end 154.94 101.6) (width 0.254) (layer F.Cu) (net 5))
 (segment (start 156.73 98.07) (end 156.73 99.81) (width 0.254) (layer F.Cu) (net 5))
 (segment (start 156.23 97.77) (end 152.4 101.6) (width 0.254) (layer F.Cu) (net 6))
 (segment (start 155.93 97.27) (end 155.13 97.27) (width 0.254) (layer F.Cu) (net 7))
 (segment (start 155.13 97.27) (end 152.4 100) (width 0.254) (layer F.Cu) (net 7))
 (segment (start 151.46 100) (end 149.86 101.6) (width 0.254) (layer F.Cu) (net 7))
 (segment (start 152.4 100) (end 151.46 100) (width 0.254) (layer F.Cu) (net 7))
 (segment (start 151.12 92.7) (end 149.86 91.44) (width 0.254) (layer F.Cu) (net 8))
 (segment (start 152.8 92.7) (end 151.12 92.7) (width 0.254) (layer F.Cu) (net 8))
 (segment (start 153.8 93.7) (end 152.8 92.7) (width 0.254) (layer F.Cu) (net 8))
 (segment (start 153.8 95.7) (end 153.8 93.7) (width 0.254) (layer F.Cu) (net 8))
 (segment (start 155.93 96.77) (end 154.87 96.77) (width 0.254) (layer F.Cu) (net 8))
 (segment (start 154.87 96.77) (end 153.8 95.7) (width 0.254) (layer F.Cu) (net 8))
 (segment (start 155.17 96.27) (end 155.93 96.27) (width 0.254) (layer F.Cu) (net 9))
 (segment (start 154.3 95.4) (end 155.17 96.27) (width 0.254) (layer F.Cu) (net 9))
 (segment (start 152.4 91.44) (end 154.3 93.34) (width 0.254) (layer F.Cu) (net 9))
 (segment (start 154.3 93.34) (end 154.3 95.4) (width 0.254) (layer F.Cu) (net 9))
 (segment (start 154.94 93.98) (end 154.94 91.44) (width 0.254) (layer F.Cu) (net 10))
 (segment (start 156.23 95.27) (end 154.94 93.98) (width 0.254) (layer F.Cu) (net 10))
 (segment (start 156.73 92.19) (end 157.48 91.44) (width 0.254) (layer F.Cu) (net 11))
 (segment (start 156.73 94.97) (end 156.73 92.19) (width 0.254) (layer F.Cu) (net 11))
 (segment (start 157.23 94.97) (end 157.23 93.87) (width 0.254) (layer F.Cu) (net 12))
 (segment (start 157.23 93.87) (end 158.5 92.6) (width 0.254) (layer F.Cu) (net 12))
 (segment (start 158.86 92.6) (end 158.5 92.6) (width 0.254) (layer F.Cu) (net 12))
 (segment (start 160.02 91.44) (end 158.86 92.6) (width 0.254) (layer F.Cu) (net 12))
 (segment (start 157.73 94.07) (end 158.7 93.1) (width 0.254) (layer F.Cu) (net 13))
 (segment (start 157.73 94.97) (end 157.73 94.07) (width 0.254) (layer F.Cu) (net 13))
 (segment (start 158.7 93.1) (end 160.9 93.1) (width 0.254) (layer F.Cu) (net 13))
 (segment (start 160.9 93.1) (end 162.56 91.44) (width 0.254) (layer F.Cu) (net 13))
 (segment (start 163.34 93.2) (end 165.1 91.44) (width 0.254) (layer F.Cu) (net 14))
 (segment (start 161.5 93.2) (end 163.34 93.2) (width 0.254) (layer F.Cu) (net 14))
 (segment (start 161.1 93.6) (end 161.5 93.2) (width 0.254) (layer F.Cu) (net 14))
 (segment (start 158.9 93.6) (end 161.1 93.6) (width 0.254) (layer F.Cu) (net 14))
 (segment (start 158.23 94.97) (end 158.23 94.27) (width 0.254) (layer F.Cu) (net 14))
 (segment (start 158.23 94.27) (end 158.9 93.6) (width 0.254) (layer F.Cu) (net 14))
 (segment (start 167.64 95.25) (end 167.64 99.06) (width 0.254) (layer F.Cu) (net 15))
 (segment (start 167.64 91.44) (end 167.64 93.74) (width 0.254) (layer F.Cu) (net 15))
 (segment (start 159.9 94.1) (end 158.73 95.27) (width 0.254) (layer F.Cu) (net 15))
 (segment (start 167.64 93.74) (end 167.64 95.25) (width 0.254) (layer F.Cu) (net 15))
 (segment (start 167.64 93.74) (end 167.6 93.7) (width 0.254) (layer F.Cu) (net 15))
 (segment (start 167.6 93.7) (end 161.7 93.7) (width 0.254) (layer F.Cu) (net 15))
 (segment (start 161.7 93.7) (end 161.3 94.1) (width 0.254) (layer F.Cu) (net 15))
 (segment (start 161.3 94.1) (end 159.9 94.1) (width 0.254) (layer F.Cu) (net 15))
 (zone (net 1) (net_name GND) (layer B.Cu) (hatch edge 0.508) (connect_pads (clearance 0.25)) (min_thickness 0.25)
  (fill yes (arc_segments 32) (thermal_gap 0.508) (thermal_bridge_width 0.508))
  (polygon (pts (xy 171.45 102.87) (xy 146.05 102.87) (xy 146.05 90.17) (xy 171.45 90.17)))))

